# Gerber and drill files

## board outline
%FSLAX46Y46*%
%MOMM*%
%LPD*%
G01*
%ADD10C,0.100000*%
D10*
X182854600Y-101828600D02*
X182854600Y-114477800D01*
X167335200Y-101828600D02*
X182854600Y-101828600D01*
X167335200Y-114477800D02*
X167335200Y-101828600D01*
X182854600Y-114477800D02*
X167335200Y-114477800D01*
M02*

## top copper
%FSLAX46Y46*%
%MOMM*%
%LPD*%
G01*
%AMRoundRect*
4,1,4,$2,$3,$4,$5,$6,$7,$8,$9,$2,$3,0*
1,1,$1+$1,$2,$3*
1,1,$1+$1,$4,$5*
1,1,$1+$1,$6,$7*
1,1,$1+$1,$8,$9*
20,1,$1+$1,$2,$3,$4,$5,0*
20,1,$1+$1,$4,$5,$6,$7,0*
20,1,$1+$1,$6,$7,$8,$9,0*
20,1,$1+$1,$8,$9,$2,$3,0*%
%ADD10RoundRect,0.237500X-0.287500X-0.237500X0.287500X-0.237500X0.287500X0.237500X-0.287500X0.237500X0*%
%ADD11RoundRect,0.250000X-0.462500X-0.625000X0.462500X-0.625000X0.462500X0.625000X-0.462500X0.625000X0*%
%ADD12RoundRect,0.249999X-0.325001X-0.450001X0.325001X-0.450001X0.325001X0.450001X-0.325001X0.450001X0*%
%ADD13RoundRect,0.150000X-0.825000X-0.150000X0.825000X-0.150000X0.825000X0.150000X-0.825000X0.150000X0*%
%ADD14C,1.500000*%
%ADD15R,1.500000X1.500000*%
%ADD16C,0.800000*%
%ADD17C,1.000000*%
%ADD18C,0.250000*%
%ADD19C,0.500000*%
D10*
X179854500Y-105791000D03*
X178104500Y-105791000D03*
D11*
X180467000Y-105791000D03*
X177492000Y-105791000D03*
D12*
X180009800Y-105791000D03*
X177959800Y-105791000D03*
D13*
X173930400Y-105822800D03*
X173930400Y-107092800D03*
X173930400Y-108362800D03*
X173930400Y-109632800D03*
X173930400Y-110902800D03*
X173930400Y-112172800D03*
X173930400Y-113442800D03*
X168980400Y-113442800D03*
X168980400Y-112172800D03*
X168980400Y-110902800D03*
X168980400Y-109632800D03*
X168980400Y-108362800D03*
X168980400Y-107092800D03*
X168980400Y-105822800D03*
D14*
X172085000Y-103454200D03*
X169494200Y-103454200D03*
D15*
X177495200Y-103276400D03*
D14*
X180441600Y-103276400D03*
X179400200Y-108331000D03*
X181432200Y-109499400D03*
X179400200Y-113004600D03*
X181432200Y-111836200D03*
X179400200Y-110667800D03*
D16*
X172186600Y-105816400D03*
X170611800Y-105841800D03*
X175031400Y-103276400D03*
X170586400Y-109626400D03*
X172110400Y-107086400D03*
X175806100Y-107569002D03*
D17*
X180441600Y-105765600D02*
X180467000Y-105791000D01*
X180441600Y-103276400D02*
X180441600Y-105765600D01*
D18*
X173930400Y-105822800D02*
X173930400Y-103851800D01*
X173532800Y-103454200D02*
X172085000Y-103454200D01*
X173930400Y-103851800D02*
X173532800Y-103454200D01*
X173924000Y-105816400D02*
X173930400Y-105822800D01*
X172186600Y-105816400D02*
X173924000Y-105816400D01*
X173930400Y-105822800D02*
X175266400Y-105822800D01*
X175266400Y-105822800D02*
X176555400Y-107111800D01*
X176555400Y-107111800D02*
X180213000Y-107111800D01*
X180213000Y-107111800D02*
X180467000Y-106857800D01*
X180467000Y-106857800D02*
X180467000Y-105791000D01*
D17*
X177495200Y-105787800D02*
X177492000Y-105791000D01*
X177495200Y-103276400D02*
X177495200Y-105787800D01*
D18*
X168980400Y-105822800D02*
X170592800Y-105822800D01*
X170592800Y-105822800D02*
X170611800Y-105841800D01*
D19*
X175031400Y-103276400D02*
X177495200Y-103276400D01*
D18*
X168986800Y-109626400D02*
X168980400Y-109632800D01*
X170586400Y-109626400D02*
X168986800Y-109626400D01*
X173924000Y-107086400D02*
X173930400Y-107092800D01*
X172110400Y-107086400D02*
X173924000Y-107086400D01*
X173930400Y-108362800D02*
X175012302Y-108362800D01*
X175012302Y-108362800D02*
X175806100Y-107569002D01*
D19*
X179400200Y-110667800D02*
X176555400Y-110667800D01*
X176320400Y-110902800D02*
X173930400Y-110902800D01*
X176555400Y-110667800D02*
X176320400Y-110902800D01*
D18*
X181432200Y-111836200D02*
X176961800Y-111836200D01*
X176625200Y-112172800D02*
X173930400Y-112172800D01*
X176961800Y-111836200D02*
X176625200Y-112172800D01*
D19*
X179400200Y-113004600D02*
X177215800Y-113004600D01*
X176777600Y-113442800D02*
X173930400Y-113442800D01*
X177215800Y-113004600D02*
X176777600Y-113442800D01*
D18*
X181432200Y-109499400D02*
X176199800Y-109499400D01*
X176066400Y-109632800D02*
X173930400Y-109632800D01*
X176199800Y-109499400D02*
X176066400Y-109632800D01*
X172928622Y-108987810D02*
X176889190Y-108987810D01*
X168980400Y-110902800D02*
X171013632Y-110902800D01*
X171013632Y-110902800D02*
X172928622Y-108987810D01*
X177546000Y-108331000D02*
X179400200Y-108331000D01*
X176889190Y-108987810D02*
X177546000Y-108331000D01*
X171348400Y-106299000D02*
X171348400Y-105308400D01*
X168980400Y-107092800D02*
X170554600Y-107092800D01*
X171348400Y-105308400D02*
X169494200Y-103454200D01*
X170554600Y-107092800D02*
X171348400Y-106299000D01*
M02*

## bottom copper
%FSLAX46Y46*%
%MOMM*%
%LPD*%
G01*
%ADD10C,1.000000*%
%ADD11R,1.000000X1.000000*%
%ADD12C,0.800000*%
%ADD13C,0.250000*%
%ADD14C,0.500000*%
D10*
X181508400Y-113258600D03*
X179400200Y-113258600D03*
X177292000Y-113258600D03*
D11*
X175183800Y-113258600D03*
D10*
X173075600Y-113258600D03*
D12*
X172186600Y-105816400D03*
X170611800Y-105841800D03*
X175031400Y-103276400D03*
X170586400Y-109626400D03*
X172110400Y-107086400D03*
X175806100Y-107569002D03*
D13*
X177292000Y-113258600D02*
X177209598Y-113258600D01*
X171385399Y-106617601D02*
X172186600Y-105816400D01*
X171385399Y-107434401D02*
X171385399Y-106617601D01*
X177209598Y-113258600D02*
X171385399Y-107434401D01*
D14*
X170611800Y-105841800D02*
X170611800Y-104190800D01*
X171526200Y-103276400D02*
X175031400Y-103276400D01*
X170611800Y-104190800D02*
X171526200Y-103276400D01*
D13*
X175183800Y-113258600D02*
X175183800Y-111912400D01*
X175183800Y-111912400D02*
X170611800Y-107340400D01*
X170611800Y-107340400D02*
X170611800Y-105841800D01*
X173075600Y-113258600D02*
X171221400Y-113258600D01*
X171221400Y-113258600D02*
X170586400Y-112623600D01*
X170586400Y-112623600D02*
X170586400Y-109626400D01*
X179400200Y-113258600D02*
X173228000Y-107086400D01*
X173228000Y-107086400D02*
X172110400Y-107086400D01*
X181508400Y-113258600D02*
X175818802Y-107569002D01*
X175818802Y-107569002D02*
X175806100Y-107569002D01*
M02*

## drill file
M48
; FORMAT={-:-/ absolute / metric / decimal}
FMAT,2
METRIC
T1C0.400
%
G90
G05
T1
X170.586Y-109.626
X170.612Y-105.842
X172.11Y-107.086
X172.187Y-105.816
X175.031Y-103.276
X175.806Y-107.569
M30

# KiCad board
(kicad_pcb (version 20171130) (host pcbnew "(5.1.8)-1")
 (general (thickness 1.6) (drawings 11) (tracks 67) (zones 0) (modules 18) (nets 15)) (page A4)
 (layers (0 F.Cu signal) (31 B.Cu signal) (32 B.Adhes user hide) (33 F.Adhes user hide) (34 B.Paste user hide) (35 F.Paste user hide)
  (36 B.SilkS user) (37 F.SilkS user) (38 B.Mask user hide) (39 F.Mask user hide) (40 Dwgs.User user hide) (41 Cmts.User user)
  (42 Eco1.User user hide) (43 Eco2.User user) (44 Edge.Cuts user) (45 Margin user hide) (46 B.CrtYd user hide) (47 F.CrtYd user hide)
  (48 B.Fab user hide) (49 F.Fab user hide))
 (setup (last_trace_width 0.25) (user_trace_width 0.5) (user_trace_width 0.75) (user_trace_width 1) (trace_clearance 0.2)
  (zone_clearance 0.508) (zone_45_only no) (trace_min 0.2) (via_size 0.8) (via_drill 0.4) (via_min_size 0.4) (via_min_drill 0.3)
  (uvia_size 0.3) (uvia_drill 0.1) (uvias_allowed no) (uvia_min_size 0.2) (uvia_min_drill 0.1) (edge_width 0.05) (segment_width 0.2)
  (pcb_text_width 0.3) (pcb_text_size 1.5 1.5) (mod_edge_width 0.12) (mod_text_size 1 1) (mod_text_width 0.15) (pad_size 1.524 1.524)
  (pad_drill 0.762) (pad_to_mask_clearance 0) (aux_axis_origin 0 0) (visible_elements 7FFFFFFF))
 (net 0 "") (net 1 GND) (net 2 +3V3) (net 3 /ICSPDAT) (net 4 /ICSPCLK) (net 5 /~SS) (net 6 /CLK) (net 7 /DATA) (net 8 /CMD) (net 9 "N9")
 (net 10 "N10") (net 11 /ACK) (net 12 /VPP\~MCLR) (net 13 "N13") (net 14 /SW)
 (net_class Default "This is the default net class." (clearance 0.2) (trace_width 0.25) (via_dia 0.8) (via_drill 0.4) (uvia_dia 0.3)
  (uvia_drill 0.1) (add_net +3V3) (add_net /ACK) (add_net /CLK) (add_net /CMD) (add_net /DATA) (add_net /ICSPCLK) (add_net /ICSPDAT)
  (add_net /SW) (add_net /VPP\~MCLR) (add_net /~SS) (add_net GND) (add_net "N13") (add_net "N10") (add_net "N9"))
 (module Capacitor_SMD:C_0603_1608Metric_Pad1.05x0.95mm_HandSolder (layer F.Cu) (at 178.9795 105.791)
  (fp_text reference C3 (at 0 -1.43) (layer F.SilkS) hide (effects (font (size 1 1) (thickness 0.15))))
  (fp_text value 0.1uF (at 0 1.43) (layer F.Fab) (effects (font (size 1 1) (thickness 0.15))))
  (pad 2 smd roundrect (at 0.875 0) (size 1.05 0.95) (layers F.Cu F.Paste F.Mask) (roundrect_rratio 0.25) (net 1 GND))
  (pad 1 smd roundrect (at -0.875 0) (size 1.05 0.95) (layers F.Cu F.Paste F.Mask) (roundrect_rratio 0.25) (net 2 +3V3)))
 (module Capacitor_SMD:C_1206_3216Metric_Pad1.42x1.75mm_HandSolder (layer F.Cu) (at 178.9795 105.791)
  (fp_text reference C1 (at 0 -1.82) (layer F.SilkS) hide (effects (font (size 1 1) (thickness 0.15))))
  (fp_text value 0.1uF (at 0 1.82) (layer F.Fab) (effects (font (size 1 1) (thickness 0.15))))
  (pad 2 smd roundrect (at 1.4875 0) (size 1.425 1.75) (layers F.Cu F.Paste F.Mask) (roundrect_rratio 0.1754385964912281) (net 1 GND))
  (pad 1 smd roundrect (at -1.4875 0) (size 1.425 1.75) (layers F.Cu F.Paste F.Mask) (roundrect_rratio 0.1754385964912281) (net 2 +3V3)))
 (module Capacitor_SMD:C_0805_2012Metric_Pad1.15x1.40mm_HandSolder (layer F.Cu) (at 178.9848 105.791)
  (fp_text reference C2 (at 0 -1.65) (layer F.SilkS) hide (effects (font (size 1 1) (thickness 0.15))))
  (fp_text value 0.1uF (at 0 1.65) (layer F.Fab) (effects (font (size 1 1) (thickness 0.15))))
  (pad 2 smd roundrect (at 1.025 0) (size 1.15 1.4) (layers F.Cu F.Paste F.Mask) (roundrect_rratio 0.2173904347826087) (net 1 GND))
  (pad 1 smd roundrect (at -1.025 0) (size 1.15 1.4) (layers F.Cu F.Paste F.Mask) (roundrect_rratio 0.2173904347826087) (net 2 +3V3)))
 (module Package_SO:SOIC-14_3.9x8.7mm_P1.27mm (layer F.Cu) (at 171.4554 109.6328)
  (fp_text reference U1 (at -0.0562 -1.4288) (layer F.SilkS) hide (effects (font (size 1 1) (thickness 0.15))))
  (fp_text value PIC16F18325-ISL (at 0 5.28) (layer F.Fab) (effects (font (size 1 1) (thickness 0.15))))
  (pad 14 smd roundrect (at 2.475 -3.81) (size 1.95 0.6) (layers F.Cu F.Paste F.Mask) (roundrect_rratio 0.25) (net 1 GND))
  (pad 13 smd roundrect (at 2.475 -2.54) (size 1.95 0.6) (layers F.Cu F.Paste F.Mask) (roundrect_rratio 0.25) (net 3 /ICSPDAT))
  (pad 12 smd roundrect (at 2.475 -1.27) (size 1.95 0.6) (layers F.Cu F.Paste F.Mask) (roundrect_rratio 0.25) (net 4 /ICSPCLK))
  (pad 11 smd roundrect (at 2.475 0) (size 1.95 0.6) (layers F.Cu F.Paste F.Mask) (roundrect_rratio 0.25) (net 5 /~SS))
  (pad 10 smd roundrect (at 2.475 1.27) (size 1.95 0.6) (layers F.Cu F.Paste F.Mask) (roundrect_rratio 0.25) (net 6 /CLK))
  (pad 9 smd roundrect (at 2.475 2.54) (size 1.95 0.6) (layers F.Cu F.Paste F.Mask) (roundrect_rratio 0.25) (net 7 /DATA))
  (pad 8 smd roundrect (at 2.475 3.81) (size 1.95 0.6) (layers F.Cu F.Paste F.Mask) (roundrect_rratio 0.25) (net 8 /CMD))
  (pad 7 smd roundrect (at -2.475 3.81) (size 1.95 0.6) (layers F.Cu F.Paste F.Mask) (roundrect_rratio 0.25) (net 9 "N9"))
  (pad 6 smd roundrect (at -2.475 2.54) (size 1.95 0.6) (layers F.Cu F.Paste F.Mask) (roundrect_rratio 0.25) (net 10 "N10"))
  (pad 5 smd roundrect (at -2.475 1.27) (size 1.95 0.6) (layers F.Cu F.Paste F.Mask) (roundrect_rratio 0.25) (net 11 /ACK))
  (pad 4 smd roundrect (at -2.475 0) (size 1.95 0.6) (layers F.Cu F.Paste F.Mask) (roundrect_rratio 0.25) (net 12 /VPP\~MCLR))
  (pad 3 smd roundrect (at -2.475 -1.27) (size 1.95 0.6) (layers F.Cu F.Paste F.Mask) (roundrect_rratio 0.25) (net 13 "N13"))
  (pad 2 smd roundrect (at -2.475 -2.54) (size 1.95 0.6) (layers F.Cu F.Paste F.Mask) (roundrect_rratio 0.25) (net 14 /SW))
  (pad 1 smd roundrect (at -2.475 -3.81) (size 1.95 0.6) (layers F.Cu F.Paste F.Mask) (roundrect_rratio 0.25) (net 2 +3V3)))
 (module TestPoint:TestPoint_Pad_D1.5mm (layer F.Cu) (at 172.085 103.4542 90)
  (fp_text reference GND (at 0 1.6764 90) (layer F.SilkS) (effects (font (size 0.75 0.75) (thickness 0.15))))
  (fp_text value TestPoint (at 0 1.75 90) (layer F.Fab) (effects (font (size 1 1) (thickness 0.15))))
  (pad 1 smd circle (at 0 0 90) (size 1.5 1.5) (layers F.Cu F.Mask) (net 1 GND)))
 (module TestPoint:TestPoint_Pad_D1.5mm (layer F.Cu) (at 169.4942 103.4542 90)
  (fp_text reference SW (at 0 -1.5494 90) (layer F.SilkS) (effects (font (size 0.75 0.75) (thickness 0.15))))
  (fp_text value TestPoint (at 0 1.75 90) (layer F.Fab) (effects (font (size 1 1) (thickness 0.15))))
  (pad 1 smd circle (at 0 0 90) (size 1.5 1.5) (layers F.Cu F.Mask) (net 14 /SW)))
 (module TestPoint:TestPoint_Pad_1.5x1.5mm (layer F.Cu) (at 177.4952 103.2764 180)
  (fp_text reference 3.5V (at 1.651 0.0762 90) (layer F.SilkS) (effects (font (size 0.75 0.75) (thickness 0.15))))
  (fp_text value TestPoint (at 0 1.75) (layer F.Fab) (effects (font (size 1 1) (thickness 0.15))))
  (pad 1 smd rect (at 0 0 180) (size 1.5 1.5) (layers F.Cu F.Mask) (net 2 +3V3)))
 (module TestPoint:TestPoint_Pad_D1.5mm (layer F.Cu) (at 180.4416 103.2764)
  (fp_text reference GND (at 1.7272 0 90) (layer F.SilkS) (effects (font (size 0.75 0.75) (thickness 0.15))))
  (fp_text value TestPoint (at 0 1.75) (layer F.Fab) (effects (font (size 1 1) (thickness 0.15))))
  (pad 1 smd circle (at 0 0) (size 1.5 1.5) (layers F.Cu F.Mask) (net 1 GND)))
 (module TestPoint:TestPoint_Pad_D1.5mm (layer F.Cu) (at 179.4002 108.331)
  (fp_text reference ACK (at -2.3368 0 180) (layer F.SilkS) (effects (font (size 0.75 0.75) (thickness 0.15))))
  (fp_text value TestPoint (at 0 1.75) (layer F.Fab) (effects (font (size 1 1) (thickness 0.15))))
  (pad 1 smd circle (at 0 0) (size 1.5 1.5) (layers F.Cu F.Mask) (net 11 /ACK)))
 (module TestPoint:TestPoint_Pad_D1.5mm (layer F.Cu) (at 181.4322 109.4994)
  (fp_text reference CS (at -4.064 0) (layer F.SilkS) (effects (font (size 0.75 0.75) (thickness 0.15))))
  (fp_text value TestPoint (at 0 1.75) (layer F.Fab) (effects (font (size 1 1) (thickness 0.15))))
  (pad 1 smd circle (at 0 0) (size 1.5 1.5) (layers F.Cu F.Mask) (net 5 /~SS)))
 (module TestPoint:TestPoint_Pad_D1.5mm (layer F.Cu) (at 179.4002 113.0046)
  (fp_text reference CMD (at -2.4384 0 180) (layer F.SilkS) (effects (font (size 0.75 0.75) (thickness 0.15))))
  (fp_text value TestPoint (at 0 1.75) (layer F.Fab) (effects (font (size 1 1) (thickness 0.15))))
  (pad 1 smd circle (at 0 0) (size 1.5 1.5) (layers F.Cu F.Mask) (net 8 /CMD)))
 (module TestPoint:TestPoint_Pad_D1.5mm (layer F.Cu) (at 181.4322 111.8362)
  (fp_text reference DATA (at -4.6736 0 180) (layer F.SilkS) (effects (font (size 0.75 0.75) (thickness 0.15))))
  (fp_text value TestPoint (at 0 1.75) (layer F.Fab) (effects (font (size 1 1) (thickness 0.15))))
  (pad 1 smd circle (at 0 0) (size 1.5 1.5) (layers F.Cu F.Mask) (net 7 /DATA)))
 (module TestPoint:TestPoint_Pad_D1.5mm (layer F.Cu) (at 179.4002 110.6678)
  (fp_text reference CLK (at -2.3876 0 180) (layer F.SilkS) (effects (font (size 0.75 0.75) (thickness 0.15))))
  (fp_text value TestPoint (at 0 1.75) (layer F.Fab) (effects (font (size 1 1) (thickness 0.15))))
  (pad 1 smd circle (at 0 0) (size 1.5 1.5) (layers F.Cu F.Mask) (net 6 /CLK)))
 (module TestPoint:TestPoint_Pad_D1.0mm (layer B.Cu) (at 181.5084 113.2586 180)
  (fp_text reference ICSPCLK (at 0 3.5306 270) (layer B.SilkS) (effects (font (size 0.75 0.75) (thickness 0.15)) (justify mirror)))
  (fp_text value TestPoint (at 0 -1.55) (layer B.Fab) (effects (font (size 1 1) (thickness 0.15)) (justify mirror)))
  (pad 1 smd circle (at 0 0 180) (size 1 1) (layers B.Cu B.Mask) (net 4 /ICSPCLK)))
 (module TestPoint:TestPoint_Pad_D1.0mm (layer B.Cu) (at 179.4002 113.2586 180)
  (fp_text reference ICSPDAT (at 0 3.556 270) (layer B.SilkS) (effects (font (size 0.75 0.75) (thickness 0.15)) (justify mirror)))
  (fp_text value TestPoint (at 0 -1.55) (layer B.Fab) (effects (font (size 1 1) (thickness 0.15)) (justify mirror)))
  (pad 1 smd circle (at 0 0 180) (size 1 1) (layers B.Cu B.Mask) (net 3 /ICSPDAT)))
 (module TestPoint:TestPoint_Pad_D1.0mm (layer B.Cu) (at 177.292 113.2586 180)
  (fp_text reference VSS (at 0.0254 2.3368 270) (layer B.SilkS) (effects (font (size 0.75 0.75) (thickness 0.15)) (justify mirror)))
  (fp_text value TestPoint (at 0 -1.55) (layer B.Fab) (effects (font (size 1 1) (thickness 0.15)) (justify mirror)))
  (pad 1 smd circle (at 0 0 180) (size 1 1) (layers B.Cu B.Mask) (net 1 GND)))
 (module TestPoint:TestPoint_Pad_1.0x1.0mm (layer B.Cu) (at 175.1838 113.2586 180)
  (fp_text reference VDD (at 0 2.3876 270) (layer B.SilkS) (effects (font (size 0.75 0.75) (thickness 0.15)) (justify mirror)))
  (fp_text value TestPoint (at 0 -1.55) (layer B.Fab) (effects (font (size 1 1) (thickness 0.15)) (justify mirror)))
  (pad 1 smd rect (at 0 0 180) (size 1 1) (layers B.Cu B.Mask) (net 2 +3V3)))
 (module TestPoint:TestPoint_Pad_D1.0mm (layer B.Cu) (at 173.0756 113.2586 180)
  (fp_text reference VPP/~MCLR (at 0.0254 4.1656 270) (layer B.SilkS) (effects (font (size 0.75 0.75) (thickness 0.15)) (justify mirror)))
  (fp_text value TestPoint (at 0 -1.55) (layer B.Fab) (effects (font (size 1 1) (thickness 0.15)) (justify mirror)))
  (pad 1 smd circle (at 0 0 180) (size 1 1) (layers B.Cu B.Mask) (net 12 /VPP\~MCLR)))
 (gr_line (start 182.8546 101.8286) (end 182.8546 114.4778) (layer Edge.Cuts) (width 0.1))
 (gr_line (start 167.3352 101.8286) (end 182.8546 101.8286) (layer Edge.Cuts) (width 0.1))
 (gr_line (start 167.3352 114.4778) (end 167.3352 101.8286) (layer Edge.Cuts) (width 0.1))
 (gr_line (start 182.8546 114.4778) (end 167.3352 114.4778) (layer Edge.Cuts) (width 0.1))
 (segment (start 180.4416 105.7656) (end 180.467 105.791) (width 1) (layer F.Cu) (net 1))
 (segment (start 180.4416 103.2764) (end 180.4416 105.7656) (width 1) (layer F.Cu) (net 1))
 (segment (start 173.9304 105.8228) (end 173.9304 103.8518) (width 0.25) (layer F.Cu) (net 1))
 (segment (start 173.5328 103.4542) (end 172.085 103.4542) (width 0.25) (layer F.Cu) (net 1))
 (segment (start 173.9304 103.8518) (end 173.5328 103.4542) (width 0.25) (layer F.Cu) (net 1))
 (via (at 172.1866 105.8164) (size 0.8) (drill 0.4) (layers F.Cu B.Cu) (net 1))
 (segment (start 177.292 113.2586) (end 177.209598 113.2586) (width 0.25) (layer B.Cu) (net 1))
 (segment (start 171.385399 106.617601) (end 172.1866 105.8164) (width 0.25) (layer B.Cu) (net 1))
 (segment (start 171.385399 107.434401) (end 171.385399 106.617601) (width 0.25) (layer B.Cu) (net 1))
 (segment (start 177.209598 113.2586) (end 171.385399 107.434401) (width 0.25) (layer B.Cu) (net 1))
 (segment (start 173.924 105.8164) (end 173.9304 105.8228) (width 0.25) (layer F.Cu) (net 1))
 (segment (start 172.1866 105.8164) (end 173.924 105.8164) (width 0.25) (layer F.Cu) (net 1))
 (segment (start 173.9304 105.8228) (end 175.2664 105.8228) (width 0.25) (layer F.Cu) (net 1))
 (segment (start 175.2664 105.8228) (end 176.5554 107.1118) (width 0.25) (layer F.Cu) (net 1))
 (segment (start 176.5554 107.1118) (end 180.213 107.1118) (width 0.25) (layer F.Cu) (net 1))
 (segment (start 180.213 107.1118) (end 180.467 106.8578) (width 0.25) (layer F.Cu) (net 1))
 (segment (start 180.467 106.8578) (end 180.467 105.791) (width 0.25) (layer F.Cu) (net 1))
 (segment (start 177.4952 105.7878) (end 177.492 105.791) (width 1) (layer F.Cu) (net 2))
 (segment (start 177.4952 103.2764) (end 177.4952 105.7878) (width 1) (layer F.Cu) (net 2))
 (via (at 170.6118 105.8418) (size 0.8) (drill 0.4) (layers F.Cu B.Cu) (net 2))
 (segment (start 168.9804 105.8228) (end 170.5928 105.8228) (width 0.25) (layer F.Cu) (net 2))
 (segment (start 170.5928 105.8228) (end 170.6118 105.8418) (width 0.25) (layer F.Cu) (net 2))
 (via (at 175.0314 103.2764) (size 0.8) (drill 0.4) (layers F.Cu B.Cu) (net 2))
 (segment (start 175.0314 103.2764) (end 177.4952 103.2764) (width 0.5) (layer F.Cu) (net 2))
 (segment (start 170.6118 105.8418) (end 170.6118 104.1908) (width 0.5) (layer B.Cu) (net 2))
 (segment (start 171.5262 103.2764) (end 175.0314 103.2764) (width 0.5) (layer B.Cu) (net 2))
 (segment (start 170.6118 104.1908) (end 171.5262 103.2764) (width 0.5) (layer B.Cu) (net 2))
 (segment (start 175.1838 113.2586) (end 175.1838 111.9124) (width 0.25) (layer B.Cu) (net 2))
 (segment (start 175.1838 111.9124) (end 170.6118 107.3404) (width 0.25) (layer B.Cu) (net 2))
 (segment (start 170.6118 107.3404) (end 170.6118 105.8418) (width 0.25) (layer B.Cu) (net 2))
 (segment (start 173.0756 113.2586) (end 171.2214 113.2586) (width 0.25) (layer B.Cu) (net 12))
 (via (at 170.5864 109.6264) (size 0.8) (drill 0.4) (layers F.Cu B.Cu) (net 12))
 (segment (start 171.2214 113.2586) (end 170.5864 112.6236) (width 0.25) (layer B.Cu) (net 12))
 (segment (start 170.5864 112.6236) (end 170.5864 109.6264) (width 0.25) (layer B.Cu) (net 12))
 (segment (start 168.9868 109.6264) (end 168.9804 109.6328) (width 0.25) (layer F.Cu) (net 12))
 (segment (start 170.5864 109.6264) (end 168.9868 109.6264) (width 0.25) (layer F.Cu) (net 12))
 (segment (start 179.4002 113.2586) (end 173.228 107.0864) (width 0.25) (layer B.Cu) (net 3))
 (segment (start 173.228 107.0864) (end 172.1104 107.0864) (width 0.25) (layer B.Cu) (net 3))
 (segment (start 173.924 107.0864) (end 173.9304 107.0928) (width 0.25) (layer F.Cu) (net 3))
 (segment (start 172.1104 107.0864) (end 173.924 107.0864) (width 0.25) (layer F.Cu) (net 3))
 (via (at 172.1104 107.0864) (size 0.8) (drill 0.4) (layers F.Cu B.Cu) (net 3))
 (via (at 175.8061 107.569002) (size 0.8) (drill 0.4) (layers F.Cu B.Cu) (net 4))
 (segment (start 181.5084 113.2586) (end 175.818802 107.569002) (width 0.25) (layer B.Cu) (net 4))
 (segment (start 175.818802 107.569002) (end 175.8061 107.569002) (width 0.25) (layer B.Cu) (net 4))
 (segment (start 173.9304 108.3628) (end 175.012302 108.3628) (width 0.25) (layer F.Cu) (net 4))
 (segment (start 175.012302 108.3628) (end 175.8061 107.569002) (width 0.25) (layer F.Cu) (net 4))
 (segment (start 179.4002 110.6678) (end 176.5554 110.6678) (width 0.5) (layer F.Cu) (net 6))
 (segment (start 176.3204 110.9028) (end 173.9304 110.9028) (width 0.5) (layer F.Cu) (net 6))
 (segment (start 176.5554 110.6678) (end 176.3204 110.9028) (width 0.5) (layer F.Cu) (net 6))
 (segment (start 181.4322 111.8362) (end 176.9618 111.8362) (width 0.25) (layer F.Cu) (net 7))
 (segment (start 176.6252 112.1728) (end 173.9304 112.1728) (width 0.25) (layer F.Cu) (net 7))
 (segment (start 176.9618 111.8362) (end 176.6252 112.1728) (width 0.25) (layer F.Cu) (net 7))
 (segment (start 179.4002 113.0046) (end 177.2158 113.0046) (width 0.5) (layer F.Cu) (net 8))
 (segment (start 176.7776 113.4428) (end 173.9304 113.4428) (width 0.5) (layer F.Cu) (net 8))
 (segment (start 177.2158 113.0046) (end 176.7776 113.4428) (width 0.5) (layer F.Cu) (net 8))
 (segment (start 181.4322 109.4994) (end 176.1998 109.4994) (width 0.25) (layer F.Cu) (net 5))
 (segment (start 176.0664 109.6328) (end 173.9304 109.6328) (width 0.25) (layer F.Cu) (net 5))
 (segment (start 176.1998 109.4994) (end 176.0664 109.6328) (width 0.25) (layer F.Cu) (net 5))
 (segment (start 172.928622 108.98781) (end 176.88919 108.98781) (width 0.25) (layer F.Cu) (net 11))
 (segment (start 168.9804 110.9028) (end 171.013632 110.9028) (width 0.25) (layer F.Cu) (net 11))
 (segment (start 171.013632 110.9028) (end 172.928622 108.98781) (width 0.25) (layer F.Cu) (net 11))
 (segment (start 177.546 108.331) (end 179.4002 108.331) (width 0.25) (layer F.Cu) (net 11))
 (segment (start 176.88919 108.98781) (end 177.546 108.331) (width 0.25) (layer F.Cu) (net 11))
 (segment (start 171.3484 106.299) (end 171.3484 105.3084) (width 0.25) (layer F.Cu) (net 14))
 (segment (start 168.9804 107.0928) (end 170.5546 107.0928) (width 0.25) (layer F.Cu) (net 14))
 (segment (start 171.3484 105.3084) (end 169.4942 103.4542) (width 0.25) (layer F.Cu) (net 14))
 (segment (start 170.5546 107.0928) (end 171.3484 106.299) (width 0.25) (layer F.Cu) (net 14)))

